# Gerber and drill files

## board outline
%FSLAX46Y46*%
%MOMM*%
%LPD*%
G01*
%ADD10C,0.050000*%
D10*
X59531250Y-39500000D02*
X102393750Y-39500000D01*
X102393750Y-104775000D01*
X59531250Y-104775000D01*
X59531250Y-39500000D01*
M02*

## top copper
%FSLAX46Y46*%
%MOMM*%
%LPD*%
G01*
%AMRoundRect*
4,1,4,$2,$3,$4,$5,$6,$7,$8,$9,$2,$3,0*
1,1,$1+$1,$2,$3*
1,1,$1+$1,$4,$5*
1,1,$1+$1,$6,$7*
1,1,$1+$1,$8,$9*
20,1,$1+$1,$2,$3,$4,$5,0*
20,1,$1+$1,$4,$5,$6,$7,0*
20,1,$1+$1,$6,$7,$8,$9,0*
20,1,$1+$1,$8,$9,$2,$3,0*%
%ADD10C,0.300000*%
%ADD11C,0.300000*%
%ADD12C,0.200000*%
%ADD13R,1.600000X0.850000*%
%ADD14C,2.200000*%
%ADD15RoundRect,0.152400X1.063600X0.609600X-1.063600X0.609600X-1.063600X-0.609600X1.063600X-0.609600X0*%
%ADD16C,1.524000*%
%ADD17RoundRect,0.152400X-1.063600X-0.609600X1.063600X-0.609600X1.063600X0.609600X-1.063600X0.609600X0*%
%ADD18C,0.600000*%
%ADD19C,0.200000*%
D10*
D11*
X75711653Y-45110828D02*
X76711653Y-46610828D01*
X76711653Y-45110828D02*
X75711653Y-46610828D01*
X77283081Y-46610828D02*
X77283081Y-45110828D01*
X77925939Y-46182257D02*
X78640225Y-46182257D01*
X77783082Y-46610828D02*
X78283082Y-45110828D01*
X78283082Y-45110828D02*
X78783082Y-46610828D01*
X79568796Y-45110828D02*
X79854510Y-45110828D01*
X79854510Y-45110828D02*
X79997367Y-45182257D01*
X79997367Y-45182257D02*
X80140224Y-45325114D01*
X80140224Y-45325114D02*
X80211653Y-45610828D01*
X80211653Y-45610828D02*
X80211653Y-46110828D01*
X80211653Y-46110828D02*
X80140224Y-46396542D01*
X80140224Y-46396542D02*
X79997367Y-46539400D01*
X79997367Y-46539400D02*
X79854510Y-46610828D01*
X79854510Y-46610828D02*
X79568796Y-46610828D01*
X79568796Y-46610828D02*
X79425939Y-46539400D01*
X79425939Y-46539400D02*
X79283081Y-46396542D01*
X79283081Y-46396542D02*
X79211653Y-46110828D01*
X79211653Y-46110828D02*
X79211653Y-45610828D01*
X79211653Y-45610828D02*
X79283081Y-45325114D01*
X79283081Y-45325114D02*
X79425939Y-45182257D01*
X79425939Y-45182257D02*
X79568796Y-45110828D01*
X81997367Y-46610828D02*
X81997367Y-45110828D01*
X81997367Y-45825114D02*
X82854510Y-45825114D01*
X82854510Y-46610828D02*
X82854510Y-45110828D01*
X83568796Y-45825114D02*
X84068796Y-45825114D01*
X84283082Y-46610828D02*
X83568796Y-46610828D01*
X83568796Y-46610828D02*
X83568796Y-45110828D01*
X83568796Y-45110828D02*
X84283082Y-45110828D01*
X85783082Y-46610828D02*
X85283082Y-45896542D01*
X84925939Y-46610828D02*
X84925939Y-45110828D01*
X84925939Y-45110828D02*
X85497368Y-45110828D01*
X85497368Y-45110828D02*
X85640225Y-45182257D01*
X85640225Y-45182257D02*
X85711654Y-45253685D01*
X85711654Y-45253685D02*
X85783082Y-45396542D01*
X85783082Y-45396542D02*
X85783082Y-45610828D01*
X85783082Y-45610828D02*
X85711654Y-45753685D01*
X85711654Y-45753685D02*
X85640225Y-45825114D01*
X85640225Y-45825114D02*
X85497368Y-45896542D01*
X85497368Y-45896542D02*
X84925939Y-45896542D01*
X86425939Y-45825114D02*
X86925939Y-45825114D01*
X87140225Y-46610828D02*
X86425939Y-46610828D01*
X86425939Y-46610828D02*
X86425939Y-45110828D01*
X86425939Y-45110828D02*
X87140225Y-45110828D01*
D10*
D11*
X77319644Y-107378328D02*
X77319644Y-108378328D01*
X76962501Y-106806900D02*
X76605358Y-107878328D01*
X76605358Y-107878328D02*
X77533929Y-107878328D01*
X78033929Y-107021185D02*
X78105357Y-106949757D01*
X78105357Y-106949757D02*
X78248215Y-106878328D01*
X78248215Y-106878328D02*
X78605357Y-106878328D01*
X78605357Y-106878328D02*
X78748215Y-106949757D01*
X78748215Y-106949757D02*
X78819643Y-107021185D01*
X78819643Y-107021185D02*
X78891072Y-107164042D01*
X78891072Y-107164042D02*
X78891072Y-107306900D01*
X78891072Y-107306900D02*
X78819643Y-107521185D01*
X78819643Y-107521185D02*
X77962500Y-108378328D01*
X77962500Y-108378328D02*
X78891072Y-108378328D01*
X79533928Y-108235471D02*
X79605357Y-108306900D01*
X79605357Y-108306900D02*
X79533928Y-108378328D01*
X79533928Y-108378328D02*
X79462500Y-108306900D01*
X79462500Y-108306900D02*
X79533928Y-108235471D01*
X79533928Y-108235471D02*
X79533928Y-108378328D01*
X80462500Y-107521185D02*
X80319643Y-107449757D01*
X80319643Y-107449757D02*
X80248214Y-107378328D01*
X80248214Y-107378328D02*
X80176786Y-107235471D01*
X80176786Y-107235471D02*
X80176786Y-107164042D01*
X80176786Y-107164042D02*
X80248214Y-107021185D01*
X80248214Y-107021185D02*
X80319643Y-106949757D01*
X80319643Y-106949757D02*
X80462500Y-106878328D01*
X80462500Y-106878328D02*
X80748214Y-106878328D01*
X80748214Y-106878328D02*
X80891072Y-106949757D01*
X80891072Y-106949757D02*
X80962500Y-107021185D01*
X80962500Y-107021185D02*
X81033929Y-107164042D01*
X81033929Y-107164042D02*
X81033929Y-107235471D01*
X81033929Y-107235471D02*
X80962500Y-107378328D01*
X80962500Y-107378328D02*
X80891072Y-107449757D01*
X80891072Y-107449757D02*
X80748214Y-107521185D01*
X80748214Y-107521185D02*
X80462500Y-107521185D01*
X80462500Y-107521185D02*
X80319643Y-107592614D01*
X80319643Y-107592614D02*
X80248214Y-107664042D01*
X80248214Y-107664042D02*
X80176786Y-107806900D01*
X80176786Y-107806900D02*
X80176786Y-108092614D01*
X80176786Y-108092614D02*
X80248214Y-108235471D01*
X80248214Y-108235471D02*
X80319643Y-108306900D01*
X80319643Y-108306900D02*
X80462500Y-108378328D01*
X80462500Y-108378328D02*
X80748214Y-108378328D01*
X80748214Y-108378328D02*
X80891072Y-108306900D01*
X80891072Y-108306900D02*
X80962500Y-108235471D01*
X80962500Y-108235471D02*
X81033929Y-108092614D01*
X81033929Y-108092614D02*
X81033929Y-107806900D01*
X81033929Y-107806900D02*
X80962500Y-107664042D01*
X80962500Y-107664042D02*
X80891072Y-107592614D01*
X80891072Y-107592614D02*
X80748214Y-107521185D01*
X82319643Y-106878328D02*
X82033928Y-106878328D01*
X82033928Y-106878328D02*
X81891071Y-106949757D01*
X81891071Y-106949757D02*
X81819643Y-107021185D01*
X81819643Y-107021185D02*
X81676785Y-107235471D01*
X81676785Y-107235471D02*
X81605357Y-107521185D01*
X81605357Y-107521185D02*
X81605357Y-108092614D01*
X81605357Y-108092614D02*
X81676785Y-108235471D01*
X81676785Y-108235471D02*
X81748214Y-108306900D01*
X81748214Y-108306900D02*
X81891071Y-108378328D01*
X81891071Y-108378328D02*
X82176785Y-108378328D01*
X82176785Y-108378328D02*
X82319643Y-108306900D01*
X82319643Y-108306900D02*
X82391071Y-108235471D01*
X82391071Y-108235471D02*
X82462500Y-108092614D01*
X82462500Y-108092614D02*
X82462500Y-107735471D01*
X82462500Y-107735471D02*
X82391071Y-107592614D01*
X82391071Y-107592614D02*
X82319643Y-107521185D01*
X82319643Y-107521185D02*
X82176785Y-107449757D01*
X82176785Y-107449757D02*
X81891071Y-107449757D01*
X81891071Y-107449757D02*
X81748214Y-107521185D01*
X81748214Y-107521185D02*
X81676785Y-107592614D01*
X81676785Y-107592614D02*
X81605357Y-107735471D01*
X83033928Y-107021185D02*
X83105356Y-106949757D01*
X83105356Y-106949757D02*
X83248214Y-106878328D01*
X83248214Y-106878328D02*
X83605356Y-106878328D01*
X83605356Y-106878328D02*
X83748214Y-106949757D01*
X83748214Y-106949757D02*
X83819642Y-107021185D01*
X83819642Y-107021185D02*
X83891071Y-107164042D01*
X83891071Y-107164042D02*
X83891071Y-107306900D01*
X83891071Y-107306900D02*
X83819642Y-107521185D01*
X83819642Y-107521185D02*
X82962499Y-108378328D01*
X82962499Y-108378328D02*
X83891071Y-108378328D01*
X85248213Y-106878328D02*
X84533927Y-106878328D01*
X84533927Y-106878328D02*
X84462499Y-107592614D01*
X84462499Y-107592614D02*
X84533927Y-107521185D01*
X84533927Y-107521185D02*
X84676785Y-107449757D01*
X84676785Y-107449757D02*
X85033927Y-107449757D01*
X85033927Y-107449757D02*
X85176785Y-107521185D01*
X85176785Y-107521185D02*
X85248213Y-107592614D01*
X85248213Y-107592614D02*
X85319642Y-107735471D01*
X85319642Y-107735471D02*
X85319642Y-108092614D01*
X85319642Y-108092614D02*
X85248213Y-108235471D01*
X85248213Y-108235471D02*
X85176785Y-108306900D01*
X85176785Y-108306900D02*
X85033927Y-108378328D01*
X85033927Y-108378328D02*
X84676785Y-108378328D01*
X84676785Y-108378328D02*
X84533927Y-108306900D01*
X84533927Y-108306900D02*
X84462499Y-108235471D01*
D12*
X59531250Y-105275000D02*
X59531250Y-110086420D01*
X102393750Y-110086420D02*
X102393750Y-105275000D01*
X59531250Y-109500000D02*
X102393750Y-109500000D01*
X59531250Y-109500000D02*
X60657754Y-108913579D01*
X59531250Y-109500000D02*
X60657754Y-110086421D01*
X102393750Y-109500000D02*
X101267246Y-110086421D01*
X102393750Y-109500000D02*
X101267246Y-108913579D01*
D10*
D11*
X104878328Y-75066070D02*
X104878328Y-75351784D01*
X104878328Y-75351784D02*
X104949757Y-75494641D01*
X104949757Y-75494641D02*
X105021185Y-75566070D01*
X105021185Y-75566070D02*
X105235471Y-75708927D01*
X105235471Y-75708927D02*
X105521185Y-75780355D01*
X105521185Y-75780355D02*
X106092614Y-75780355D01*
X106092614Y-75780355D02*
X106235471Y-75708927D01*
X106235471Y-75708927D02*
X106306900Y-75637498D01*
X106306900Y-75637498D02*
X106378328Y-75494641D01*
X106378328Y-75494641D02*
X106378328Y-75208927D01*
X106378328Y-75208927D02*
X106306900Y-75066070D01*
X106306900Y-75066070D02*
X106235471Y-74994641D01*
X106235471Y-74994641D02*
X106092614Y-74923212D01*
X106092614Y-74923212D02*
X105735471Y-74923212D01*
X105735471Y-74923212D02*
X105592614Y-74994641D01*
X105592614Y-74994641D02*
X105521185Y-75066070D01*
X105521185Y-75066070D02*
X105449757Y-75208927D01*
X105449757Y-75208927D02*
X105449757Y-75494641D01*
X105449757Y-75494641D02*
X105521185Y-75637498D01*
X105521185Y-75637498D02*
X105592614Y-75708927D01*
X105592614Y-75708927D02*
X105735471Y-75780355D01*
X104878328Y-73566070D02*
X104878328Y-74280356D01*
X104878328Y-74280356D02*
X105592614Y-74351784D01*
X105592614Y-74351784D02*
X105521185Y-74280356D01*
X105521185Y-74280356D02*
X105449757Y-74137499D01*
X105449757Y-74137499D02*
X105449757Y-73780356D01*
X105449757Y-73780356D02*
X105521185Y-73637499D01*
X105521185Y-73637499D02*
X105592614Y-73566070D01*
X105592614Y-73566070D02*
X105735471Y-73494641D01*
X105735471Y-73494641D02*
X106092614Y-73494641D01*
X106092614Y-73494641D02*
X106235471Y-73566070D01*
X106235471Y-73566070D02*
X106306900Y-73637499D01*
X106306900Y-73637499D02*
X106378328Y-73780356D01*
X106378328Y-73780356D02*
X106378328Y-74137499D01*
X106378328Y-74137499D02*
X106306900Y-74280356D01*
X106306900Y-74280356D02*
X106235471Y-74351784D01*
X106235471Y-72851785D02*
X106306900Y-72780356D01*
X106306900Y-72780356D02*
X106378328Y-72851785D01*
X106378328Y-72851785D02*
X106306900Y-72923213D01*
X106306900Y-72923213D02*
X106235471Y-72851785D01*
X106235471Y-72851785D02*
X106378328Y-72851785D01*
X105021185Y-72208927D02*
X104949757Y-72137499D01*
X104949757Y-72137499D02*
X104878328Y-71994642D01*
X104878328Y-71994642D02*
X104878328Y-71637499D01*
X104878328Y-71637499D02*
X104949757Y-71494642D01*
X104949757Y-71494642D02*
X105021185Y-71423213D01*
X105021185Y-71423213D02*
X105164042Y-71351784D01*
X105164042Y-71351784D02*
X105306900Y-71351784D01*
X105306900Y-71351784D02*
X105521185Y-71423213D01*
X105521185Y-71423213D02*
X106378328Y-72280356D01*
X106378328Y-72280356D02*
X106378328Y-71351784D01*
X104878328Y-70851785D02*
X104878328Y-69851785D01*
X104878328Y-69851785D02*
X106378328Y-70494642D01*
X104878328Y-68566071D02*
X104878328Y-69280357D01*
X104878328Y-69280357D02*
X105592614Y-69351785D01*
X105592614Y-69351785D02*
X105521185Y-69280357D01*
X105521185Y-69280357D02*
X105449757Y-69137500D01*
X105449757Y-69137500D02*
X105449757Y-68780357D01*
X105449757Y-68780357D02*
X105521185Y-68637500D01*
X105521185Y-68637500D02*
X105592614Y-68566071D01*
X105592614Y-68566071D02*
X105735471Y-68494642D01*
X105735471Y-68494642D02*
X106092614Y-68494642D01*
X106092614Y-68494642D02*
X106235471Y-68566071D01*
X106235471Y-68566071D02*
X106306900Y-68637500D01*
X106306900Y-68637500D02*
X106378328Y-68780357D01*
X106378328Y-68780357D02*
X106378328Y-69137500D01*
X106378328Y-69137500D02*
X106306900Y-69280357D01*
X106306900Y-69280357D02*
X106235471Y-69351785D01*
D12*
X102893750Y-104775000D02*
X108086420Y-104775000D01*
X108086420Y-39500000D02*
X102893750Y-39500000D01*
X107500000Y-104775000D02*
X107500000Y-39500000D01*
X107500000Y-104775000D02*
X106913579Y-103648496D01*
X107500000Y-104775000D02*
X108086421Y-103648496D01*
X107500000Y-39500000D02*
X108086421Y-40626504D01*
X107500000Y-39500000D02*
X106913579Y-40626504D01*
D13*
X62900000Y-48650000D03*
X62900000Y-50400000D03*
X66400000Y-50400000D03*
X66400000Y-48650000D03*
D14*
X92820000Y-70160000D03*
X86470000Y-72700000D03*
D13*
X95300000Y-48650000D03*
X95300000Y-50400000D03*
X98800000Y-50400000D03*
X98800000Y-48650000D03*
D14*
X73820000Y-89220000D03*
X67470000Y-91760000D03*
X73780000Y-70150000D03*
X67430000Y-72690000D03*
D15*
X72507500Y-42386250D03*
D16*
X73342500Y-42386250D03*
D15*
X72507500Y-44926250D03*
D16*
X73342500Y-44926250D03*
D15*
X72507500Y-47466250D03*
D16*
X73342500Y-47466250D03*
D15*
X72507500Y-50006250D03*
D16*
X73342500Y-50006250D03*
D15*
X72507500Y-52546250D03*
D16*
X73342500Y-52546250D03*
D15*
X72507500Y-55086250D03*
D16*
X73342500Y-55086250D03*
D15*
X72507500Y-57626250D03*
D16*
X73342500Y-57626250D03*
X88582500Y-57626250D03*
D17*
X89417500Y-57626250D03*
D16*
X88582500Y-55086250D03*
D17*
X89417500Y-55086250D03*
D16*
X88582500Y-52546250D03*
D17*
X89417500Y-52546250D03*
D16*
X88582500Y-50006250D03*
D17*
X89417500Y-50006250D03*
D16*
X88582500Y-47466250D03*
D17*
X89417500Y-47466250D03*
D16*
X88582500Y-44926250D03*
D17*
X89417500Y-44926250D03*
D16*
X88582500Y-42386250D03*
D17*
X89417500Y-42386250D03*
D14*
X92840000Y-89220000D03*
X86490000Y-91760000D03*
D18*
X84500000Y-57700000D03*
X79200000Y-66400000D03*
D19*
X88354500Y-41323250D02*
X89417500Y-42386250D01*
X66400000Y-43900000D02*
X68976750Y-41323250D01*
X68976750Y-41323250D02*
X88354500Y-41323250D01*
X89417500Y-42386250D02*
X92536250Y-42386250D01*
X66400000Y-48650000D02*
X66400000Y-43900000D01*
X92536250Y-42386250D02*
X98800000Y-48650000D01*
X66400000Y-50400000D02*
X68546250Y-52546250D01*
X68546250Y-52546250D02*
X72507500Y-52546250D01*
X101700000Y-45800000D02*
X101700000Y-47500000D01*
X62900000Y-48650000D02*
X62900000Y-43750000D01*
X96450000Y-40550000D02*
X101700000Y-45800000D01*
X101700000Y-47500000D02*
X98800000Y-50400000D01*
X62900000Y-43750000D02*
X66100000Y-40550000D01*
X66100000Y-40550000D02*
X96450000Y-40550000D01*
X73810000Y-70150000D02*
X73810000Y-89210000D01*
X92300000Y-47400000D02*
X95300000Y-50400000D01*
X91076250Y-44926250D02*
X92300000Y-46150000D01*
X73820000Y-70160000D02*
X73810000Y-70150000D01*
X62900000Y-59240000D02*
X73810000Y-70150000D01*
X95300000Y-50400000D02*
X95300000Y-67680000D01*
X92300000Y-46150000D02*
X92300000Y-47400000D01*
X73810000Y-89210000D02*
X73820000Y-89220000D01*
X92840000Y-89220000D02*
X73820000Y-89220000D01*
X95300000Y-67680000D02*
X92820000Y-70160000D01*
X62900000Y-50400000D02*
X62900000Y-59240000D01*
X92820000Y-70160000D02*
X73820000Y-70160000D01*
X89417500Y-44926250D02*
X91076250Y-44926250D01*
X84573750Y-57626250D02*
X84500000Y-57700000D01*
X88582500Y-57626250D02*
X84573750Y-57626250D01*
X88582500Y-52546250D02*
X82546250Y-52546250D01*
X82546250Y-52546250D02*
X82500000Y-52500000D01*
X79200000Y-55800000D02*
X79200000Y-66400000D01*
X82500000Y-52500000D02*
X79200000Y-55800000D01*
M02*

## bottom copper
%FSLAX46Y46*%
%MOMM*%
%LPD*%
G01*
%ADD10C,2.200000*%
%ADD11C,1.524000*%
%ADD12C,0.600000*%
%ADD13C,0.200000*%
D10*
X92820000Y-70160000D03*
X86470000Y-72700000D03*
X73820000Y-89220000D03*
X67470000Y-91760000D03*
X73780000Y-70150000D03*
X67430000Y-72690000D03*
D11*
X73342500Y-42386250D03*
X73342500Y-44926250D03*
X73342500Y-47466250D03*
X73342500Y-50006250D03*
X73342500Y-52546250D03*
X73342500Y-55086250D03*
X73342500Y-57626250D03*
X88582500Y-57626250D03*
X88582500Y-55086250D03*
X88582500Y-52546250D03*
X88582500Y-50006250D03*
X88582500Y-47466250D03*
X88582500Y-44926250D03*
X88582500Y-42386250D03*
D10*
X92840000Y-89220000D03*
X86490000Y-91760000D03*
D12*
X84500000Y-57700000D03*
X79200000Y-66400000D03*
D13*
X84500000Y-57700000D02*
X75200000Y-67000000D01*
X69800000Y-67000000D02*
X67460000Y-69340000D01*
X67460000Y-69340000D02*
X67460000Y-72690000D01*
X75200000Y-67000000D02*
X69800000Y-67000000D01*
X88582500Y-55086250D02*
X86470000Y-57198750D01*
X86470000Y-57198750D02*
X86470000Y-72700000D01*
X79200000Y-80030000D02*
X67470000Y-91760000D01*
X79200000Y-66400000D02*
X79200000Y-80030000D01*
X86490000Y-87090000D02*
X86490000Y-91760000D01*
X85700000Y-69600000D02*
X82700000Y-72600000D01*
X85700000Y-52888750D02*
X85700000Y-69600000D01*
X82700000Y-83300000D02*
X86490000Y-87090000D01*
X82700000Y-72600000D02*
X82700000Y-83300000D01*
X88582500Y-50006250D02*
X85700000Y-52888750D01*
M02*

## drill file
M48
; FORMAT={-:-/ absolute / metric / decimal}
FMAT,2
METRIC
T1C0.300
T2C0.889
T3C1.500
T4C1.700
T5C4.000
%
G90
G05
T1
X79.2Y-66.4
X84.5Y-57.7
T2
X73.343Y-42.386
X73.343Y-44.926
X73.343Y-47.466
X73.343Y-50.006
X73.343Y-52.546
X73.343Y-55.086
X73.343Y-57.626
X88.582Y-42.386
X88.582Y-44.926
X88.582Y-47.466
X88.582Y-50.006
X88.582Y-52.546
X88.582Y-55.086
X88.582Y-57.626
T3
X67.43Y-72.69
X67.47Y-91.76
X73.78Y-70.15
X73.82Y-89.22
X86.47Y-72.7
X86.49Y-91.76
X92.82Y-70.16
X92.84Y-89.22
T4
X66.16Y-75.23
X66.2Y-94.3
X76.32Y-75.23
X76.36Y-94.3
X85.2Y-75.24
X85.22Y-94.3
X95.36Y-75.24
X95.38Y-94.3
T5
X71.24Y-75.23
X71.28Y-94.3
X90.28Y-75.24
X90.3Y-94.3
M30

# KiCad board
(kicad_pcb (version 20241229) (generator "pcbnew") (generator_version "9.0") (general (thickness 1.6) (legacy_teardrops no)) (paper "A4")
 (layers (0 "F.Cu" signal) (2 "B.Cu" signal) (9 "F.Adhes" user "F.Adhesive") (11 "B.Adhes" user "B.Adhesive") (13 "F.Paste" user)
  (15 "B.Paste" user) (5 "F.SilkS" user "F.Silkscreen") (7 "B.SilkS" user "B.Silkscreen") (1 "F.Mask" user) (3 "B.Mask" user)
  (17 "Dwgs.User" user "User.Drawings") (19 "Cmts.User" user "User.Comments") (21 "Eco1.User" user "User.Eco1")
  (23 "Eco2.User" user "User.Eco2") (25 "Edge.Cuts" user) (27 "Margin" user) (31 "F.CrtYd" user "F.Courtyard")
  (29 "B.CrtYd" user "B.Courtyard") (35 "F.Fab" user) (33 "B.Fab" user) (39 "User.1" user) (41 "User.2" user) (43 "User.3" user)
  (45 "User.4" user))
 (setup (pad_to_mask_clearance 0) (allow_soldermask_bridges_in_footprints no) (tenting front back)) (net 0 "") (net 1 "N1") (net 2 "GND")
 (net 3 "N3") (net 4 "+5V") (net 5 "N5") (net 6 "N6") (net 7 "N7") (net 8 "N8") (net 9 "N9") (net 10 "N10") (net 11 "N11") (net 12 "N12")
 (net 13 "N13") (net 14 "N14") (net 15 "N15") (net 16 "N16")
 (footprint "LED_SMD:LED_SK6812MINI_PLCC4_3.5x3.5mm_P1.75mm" (layer "F.Cu") (at 64.65 49.525)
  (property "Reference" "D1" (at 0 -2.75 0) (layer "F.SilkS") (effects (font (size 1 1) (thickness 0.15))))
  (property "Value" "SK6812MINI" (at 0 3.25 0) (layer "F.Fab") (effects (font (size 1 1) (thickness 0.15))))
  (pad "1" smd rect (at -1.75 -0.875) (size 1.6 0.85) (layers "F.Cu" "F.Mask" "F.Paste") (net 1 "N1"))
  (pad "2" smd rect (at -1.75 0.875) (size 1.6 0.85) (layers "F.Cu" "F.Mask" "F.Paste") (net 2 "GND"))
  (pad "3" smd rect (at 1.75 0.875) (size 1.6 0.85) (layers "F.Cu" "F.Mask" "F.Paste") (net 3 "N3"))
  (pad "4" smd rect (at 1.75 -0.875) (size 1.6 0.85) (layers "F.Cu" "F.Mask" "F.Paste") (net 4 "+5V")))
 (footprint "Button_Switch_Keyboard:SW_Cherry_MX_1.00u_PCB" (layer "F.Cu") (at 92.82 70.16)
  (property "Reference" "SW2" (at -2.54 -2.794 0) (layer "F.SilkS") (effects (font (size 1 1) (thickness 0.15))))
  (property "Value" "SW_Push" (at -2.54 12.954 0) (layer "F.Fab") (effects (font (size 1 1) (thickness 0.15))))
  (pad "" np_thru_hole circle (at -7.62 5.08) (size 1.7 1.7) (drill 1.7) (layers "*.Cu" "*.Mask"))
  (pad "" np_thru_hole circle (at -2.54 5.08) (size 4 4) (drill 4) (layers "*.Cu" "*.Mask"))
  (pad "" np_thru_hole circle (at 2.54 5.08) (size 1.7 1.7) (drill 1.7) (layers "*.Cu" "*.Mask"))
  (pad "1" thru_hole circle (at 0 0) (size 2.2 2.2) (drill 1.5) (layers "*.Cu" "*.Mask") (remove_unused_layers no) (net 2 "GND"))
  (pad "2" thru_hole circle (at -6.35 2.54) (size 2.2 2.2) (drill 1.5) (layers "*.Cu" "*.Mask") (remove_unused_layers no) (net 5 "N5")))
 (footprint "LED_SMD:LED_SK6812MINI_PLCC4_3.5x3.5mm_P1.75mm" (layer "F.Cu") (at 97.05 49.525)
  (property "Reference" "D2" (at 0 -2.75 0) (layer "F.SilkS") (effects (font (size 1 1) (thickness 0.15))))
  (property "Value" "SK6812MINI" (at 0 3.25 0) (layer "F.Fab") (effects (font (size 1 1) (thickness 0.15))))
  (pad "1" smd rect (at -1.75 -0.875) (size 1.6 0.85) (layers "F.Cu" "F.Mask" "F.Paste") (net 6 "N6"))
  (pad "2" smd rect (at -1.75 0.875) (size 1.6 0.85) (layers "F.Cu" "F.Mask" "F.Paste") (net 2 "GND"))
  (pad "3" smd rect (at 1.75 0.875) (size 1.6 0.85) (layers "F.Cu" "F.Mask" "F.Paste") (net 1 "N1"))
  (pad "4" smd rect (at 1.75 -0.875) (size 1.6 0.85) (layers "F.Cu" "F.Mask" "F.Paste") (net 4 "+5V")))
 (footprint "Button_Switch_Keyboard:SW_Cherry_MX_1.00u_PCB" (layer "F.Cu") (at 73.82 89.22)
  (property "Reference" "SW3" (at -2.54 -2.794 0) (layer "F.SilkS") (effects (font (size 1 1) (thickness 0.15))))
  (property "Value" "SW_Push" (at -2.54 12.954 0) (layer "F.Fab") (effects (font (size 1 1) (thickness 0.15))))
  (pad "" np_thru_hole circle (at -7.62 5.08) (size 1.7 1.7) (drill 1.7) (layers "*.Cu" "*.Mask"))
  (pad "" np_thru_hole circle (at -2.54 5.08) (size 4 4) (drill 4) (layers "*.Cu" "*.Mask"))
  (pad "" np_thru_hole circle (at 2.54 5.08) (size 1.7 1.7) (drill 1.7) (layers "*.Cu" "*.Mask"))
  (pad "1" thru_hole circle (at 0 0) (size 2.2 2.2) (drill 1.5) (layers "*.Cu" "*.Mask") (remove_unused_layers no) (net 2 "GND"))
  (pad "2" thru_hole circle (at -6.35 2.54) (size 2.2 2.2) (drill 1.5) (layers "*.Cu" "*.Mask") (remove_unused_layers no) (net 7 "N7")))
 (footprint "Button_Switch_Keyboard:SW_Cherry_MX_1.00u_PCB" (layer "F.Cu") (at 73.78 70.15)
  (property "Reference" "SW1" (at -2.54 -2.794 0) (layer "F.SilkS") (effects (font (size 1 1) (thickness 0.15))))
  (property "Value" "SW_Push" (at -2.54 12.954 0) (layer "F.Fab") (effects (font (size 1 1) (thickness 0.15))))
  (pad "" np_thru_hole circle (at -7.62 5.08) (size 1.7 1.7) (drill 1.7) (layers "*.Cu" "*.Mask"))
  (pad "" np_thru_hole circle (at -2.54 5.08) (size 4 4) (drill 4) (layers "*.Cu" "*.Mask"))
  (pad "" np_thru_hole circle (at 2.54 5.08) (size 1.7 1.7) (drill 1.7) (layers "*.Cu" "*.Mask"))
  (pad "1" thru_hole circle (at 0 0) (size 2.2 2.2) (drill 1.5) (layers "*.Cu" "*.Mask") (remove_unused_layers no) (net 2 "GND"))
  (pad "2" thru_hole circle (at -6.35 2.54) (size 2.2 2.2) (drill 1.5) (layers "*.Cu" "*.Mask") (remove_unused_layers no) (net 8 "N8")))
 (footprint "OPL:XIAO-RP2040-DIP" (layer "F.Cu") (at 80.9625 50.00625)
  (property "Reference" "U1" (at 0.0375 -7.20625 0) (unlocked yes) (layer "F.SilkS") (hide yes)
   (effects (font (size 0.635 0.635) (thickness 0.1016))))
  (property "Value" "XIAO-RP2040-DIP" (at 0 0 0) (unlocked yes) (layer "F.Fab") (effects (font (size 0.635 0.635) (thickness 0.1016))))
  (pad "1" smd roundrect (at -8.455 -7.62 180) (size 2.432 1.524) (layers "F.Cu" "F.Mask") (roundrect_rratio 0.1) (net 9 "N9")
   (thermal_bridge_angle 45))
  (pad "1" thru_hole circle (at -7.62 -7.62 180) (size 1.524 1.524) (drill 0.889) (layers "*.Cu" "*.Mask") (remove_unused_layers no)
   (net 9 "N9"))
  (pad "2" smd roundrect (at -8.455 -5.08 180) (size 2.432 1.524) (layers "F.Cu" "F.Mask") (roundrect_rratio 0.1) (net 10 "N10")
   (thermal_bridge_angle 45))
  (pad "2" thru_hole circle (at -7.62 -5.08 180) (size 1.524 1.524) (drill 0.889) (layers "*.Cu" "*.Mask") (remove_unused_layers no)
   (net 10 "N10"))
  (pad "3" smd roundrect (at -8.455 -2.54 180) (size 2.432 1.524) (layers "F.Cu" "F.Mask") (roundrect_rratio 0.1) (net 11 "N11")
   (thermal_bridge_angle 45))
  (pad "3" thru_hole circle (at -7.62 -2.54 180) (size 1.524 1.524) (drill 0.889) (layers "*.Cu" "*.Mask") (remove_unused_layers no)
   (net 11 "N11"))
  (pad "4" smd roundrect (at -8.455 0 180) (size 2.432 1.524) (layers "F.Cu" "F.Mask") (roundrect_rratio 0.1) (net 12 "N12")
   (thermal_bridge_angle 45))
  (pad "4" thru_hole circle (at -7.62 0 180) (size 1.524 1.524) (drill 0.889) (layers "*.Cu" "*.Mask") (remove_unused_layers no)
   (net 12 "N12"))
  (pad "5" smd roundrect (at -8.455 2.54 180) (size 2.432 1.524) (layers "F.Cu" "F.Mask") (roundrect_rratio 0.1) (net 3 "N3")
   (thermal_bridge_angle 45))
  (pad "5" thru_hole circle (at -7.62 2.54 180) (size 1.524 1.524) (drill 0.889) (layers "*.Cu" "*.Mask") (remove_unused_layers no)
   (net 3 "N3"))
  (pad "6" smd roundrect (at -8.455 5.08 180) (size 2.432 1.524) (layers "F.Cu" "F.Mask") (roundrect_rratio 0.1) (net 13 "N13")
   (thermal_bridge_angle 45))
  (pad "6" thru_hole circle (at -7.62 5.08 180) (size 1.524 1.524) (drill 0.889) (layers "*.Cu" "*.Mask") (remove_unused_layers no)
   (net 13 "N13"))
  (pad "7" smd roundrect (at -8.455 7.62 180) (size 2.432 1.524) (layers "F.Cu" "F.Mask") (roundrect_rratio 0.1) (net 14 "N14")
   (thermal_bridge_angle 45))
  (pad "7" thru_hole circle (at -7.62 7.62 180) (size 1.524 1.524) (drill 0.889) (layers "*.Cu" "*.Mask") (remove_unused_layers no)
   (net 14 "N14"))
  (pad "8" thru_hole circle (at 7.62 7.62) (size 1.524 1.524) (drill 0.889) (layers "*.Cu" "*.Mask") (remove_unused_layers no) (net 8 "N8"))
  (pad "8" smd roundrect (at 8.455 7.62) (size 2.432 1.524) (layers "F.Cu" "F.Mask") (roundrect_rratio 0.1) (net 8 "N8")
   (thermal_bridge_angle 45))
  (pad "9" thru_hole circle (at 7.62 5.08) (size 1.524 1.524) (drill 0.889) (layers "*.Cu" "*.Mask") (remove_unused_layers no) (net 5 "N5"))
  (pad "9" smd roundrect (at 8.455 5.08) (size 2.432 1.524) (layers "F.Cu" "F.Mask") (roundrect_rratio 0.1) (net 5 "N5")
   (thermal_bridge_angle 45))
  (pad "10" thru_hole circle (at 7.62 2.54) (size 1.524 1.524) (drill 0.889) (layers "*.Cu" "*.Mask") (remove_unused_layers no) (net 7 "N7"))
  (pad "10" smd roundrect (at 8.455 2.54) (size 2.432 1.524) (layers "F.Cu" "F.Mask") (roundrect_rratio 0.1) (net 7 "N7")
   (thermal_bridge_angle 45))
  (pad "11" thru_hole circle (at 7.62 0) (size 1.524 1.524) (drill 0.889) (layers "*.Cu" "*.Mask") (remove_unused_layers no) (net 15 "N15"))
  (pad "11" smd roundrect (at 8.455 0) (size 2.432 1.524) (layers "F.Cu" "F.Mask") (roundrect_rratio 0.1) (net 15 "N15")
   (thermal_bridge_angle 45))
  (pad "12" thru_hole circle (at 7.62 -2.54) (size 1.524 1.524) (drill 0.889) (layers "*.Cu" "*.Mask") (remove_unused_layers no)
   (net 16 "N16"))
  (pad "12" smd roundrect (at 8.455 -2.54) (size 2.432 1.524) (layers "F.Cu" "F.Mask") (roundrect_rratio 0.1) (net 16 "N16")
   (thermal_bridge_angle 45))
  (pad "13" thru_hole circle (at 7.62 -5.08) (size 1.524 1.524) (drill 0.889) (layers "*.Cu" "*.Mask") (remove_unused_layers no)
   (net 2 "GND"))
  (pad "13" smd roundrect (at 8.455 -5.08) (size 2.432 1.524) (layers "F.Cu" "F.Mask") (roundrect_rratio 0.1) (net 2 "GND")
   (thermal_bridge_angle 45))
  (pad "14" thru_hole circle (at 7.62 -7.62) (size 1.524 1.524) (drill 0.889) (layers "*.Cu" "*.Mask") (remove_unused_layers no)
   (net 4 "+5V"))
  (pad "14" smd roundrect (at 8.455 -7.62) (size 2.432 1.524) (layers "F.Cu" "F.Mask") (roundrect_rratio 0.1) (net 4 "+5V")
   (thermal_bridge_angle 45)))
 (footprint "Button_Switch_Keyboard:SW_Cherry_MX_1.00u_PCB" (layer "F.Cu") (at 92.84 89.22)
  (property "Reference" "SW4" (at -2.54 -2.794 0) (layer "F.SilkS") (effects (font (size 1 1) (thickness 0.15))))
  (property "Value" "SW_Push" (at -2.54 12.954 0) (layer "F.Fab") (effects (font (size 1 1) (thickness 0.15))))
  (pad "" np_thru_hole circle (at -7.62 5.08) (size 1.7 1.7) (drill 1.7) (layers "*.Cu" "*.Mask"))
  (pad "" np_thru_hole circle (at -2.54 5.08) (size 4 4) (drill 4) (layers "*.Cu" "*.Mask"))
  (pad "" np_thru_hole circle (at 2.54 5.08) (size 1.7 1.7) (drill 1.7) (layers "*.Cu" "*.Mask"))
  (pad "1" thru_hole circle (at 0 0) (size 2.2 2.2) (drill 1.5) (layers "*.Cu" "*.Mask") (remove_unused_layers no) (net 2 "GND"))
  (pad "2" thru_hole circle (at -6.35 2.54) (size 2.2 2.2) (drill 1.5) (layers "*.Cu" "*.Mask") (remove_unused_layers no) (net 15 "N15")))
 (gr_rect (start 59.53125 39.5) (end 102.39375 104.775) (stroke (width 0.05) (type default)) (fill no) (layer "Edge.Cuts"))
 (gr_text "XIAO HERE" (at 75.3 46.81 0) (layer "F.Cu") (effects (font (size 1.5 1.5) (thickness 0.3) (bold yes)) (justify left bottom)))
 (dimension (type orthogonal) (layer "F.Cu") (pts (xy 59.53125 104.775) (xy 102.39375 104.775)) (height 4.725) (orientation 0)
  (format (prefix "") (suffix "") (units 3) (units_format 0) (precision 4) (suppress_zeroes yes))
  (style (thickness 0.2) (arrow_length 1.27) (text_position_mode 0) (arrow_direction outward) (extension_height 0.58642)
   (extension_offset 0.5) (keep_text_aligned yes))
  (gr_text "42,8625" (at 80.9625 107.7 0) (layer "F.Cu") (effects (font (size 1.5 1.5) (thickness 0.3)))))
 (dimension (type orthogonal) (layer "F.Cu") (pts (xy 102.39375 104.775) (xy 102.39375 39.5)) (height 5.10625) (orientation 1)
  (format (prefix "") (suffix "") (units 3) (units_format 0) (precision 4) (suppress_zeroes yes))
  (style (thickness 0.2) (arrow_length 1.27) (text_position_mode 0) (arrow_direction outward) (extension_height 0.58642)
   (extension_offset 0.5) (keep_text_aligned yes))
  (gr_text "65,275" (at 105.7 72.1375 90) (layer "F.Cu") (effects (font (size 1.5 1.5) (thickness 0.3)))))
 (segment (start 88.3545 41.32325) (end 89.4175 42.38625) (width 0.2) (layer "F.Cu") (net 4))
 (segment (start 66.4 43.9) (end 68.97675 41.32325) (width 0.2) (layer "F.Cu") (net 4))
 (segment (start 68.97675 41.32325) (end 88.3545 41.32325) (width 0.2) (layer "F.Cu") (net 4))
 (segment (start 89.4175 42.38625) (end 92.53625 42.38625) (width 0.2) (layer "F.Cu") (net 4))
 (segment (start 66.4 48.65) (end 66.4 43.9) (width 0.2) (layer "F.Cu") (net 4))
 (segment (start 92.53625 42.38625) (end 98.8 48.65) (width 0.2) (layer "F.Cu") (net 4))
 (segment (start 66.4 50.4) (end 68.54625 52.54625) (width 0.2) (layer "F.Cu") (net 3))
 (segment (start 68.54625 52.54625) (end 72.5075 52.54625) (width 0.2) (layer "F.Cu") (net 3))
 (segment (start 101.7 45.8) (end 101.7 47.5) (width 0.2) (layer "F.Cu") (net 1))
 (segment (start 62.9 48.65) (end 62.9 43.75) (width 0.2) (layer "F.Cu") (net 1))
 (segment (start 96.45 40.55) (end 101.7 45.8) (width 0.2) (layer "F.Cu") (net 1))
 (segment (start 101.7 47.5) (end 98.8 50.4) (width 0.2) (layer "F.Cu") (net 1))
 (segment (start 62.9 43.75) (end 66.1 40.55) (width 0.2) (layer "F.Cu") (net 1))
 (segment (start 66.1 40.55) (end 96.45 40.55) (width 0.2) (layer "F.Cu") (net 1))
 (segment (start 73.81 70.15) (end 73.81 89.21) (width 0.2) (layer "F.Cu") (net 2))
 (segment (start 92.3 47.4) (end 95.3 50.4) (width 0.2) (layer "F.Cu") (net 2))
 (segment (start 91.07625 44.92625) (end 92.3 46.15) (width 0.2) (layer "F.Cu") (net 2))
 (segment (start 73.82 70.16) (end 73.81 70.15) (width 0.2) (layer "F.Cu") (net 2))
 (segment (start 62.9 59.24) (end 73.81 70.15) (width 0.2) (layer "F.Cu") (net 2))
 (segment (start 95.3 50.4) (end 95.3 67.68) (width 0.2) (layer "F.Cu") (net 2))
 (segment (start 92.3 46.15) (end 92.3 47.4) (width 0.2) (layer "F.Cu") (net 2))
 (segment (start 73.81 89.21) (end 73.82 89.22) (width 0.2) (layer "F.Cu") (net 2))
 (segment (start 92.84 89.22) (end 73.82 89.22) (width 0.2) (layer "F.Cu") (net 2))
 (segment (start 95.3 67.68) (end 92.82 70.16) (width 0.2) (layer "F.Cu") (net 2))
 (segment (start 62.9 50.4) (end 62.9 59.24) (width 0.2) (layer "F.Cu") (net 2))
 (segment (start 92.82 70.16) (end 73.82 70.16) (width 0.2) (layer "F.Cu") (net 2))
 (segment (start 89.4175 44.92625) (end 91.07625 44.92625) (width 0.2) (layer "F.Cu") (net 2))
 (segment (start 84.57375 57.62625) (end 84.5 57.7) (width 0.2) (layer "F.Cu") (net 8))
 (segment (start 88.5825 57.62625) (end 84.57375 57.62625) (width 0.2) (layer "F.Cu") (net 8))
 (via (at 84.5 57.7) (size 0.6) (drill 0.3) (layers "F.Cu" "B.Cu") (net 8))
 (segment (start 84.5 57.7) (end 75.2 67) (width 0.2) (layer "B.Cu") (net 8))
 (segment (start 69.8 67) (end 67.46 69.34) (width 0.2) (layer "B.Cu") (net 8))
 (segment (start 67.46 69.34) (end 67.46 72.69) (width 0.2) (layer "B.Cu") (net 8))
 (segment (start 75.2 67) (end 69.8 67) (width 0.2) (layer "B.Cu") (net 8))
 (segment (start 88.5825 55.08625) (end 86.47 57.19875) (width 0.2) (layer "B.Cu") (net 5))
 (segment (start 86.47 57.19875) (end 86.47 72.7) (width 0.2) (layer "B.Cu") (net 5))
 (segment (start 88.5825 52.54625) (end 82.54625 52.54625) (width 0.2) (layer "F.Cu") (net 7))
 (segment (start 82.54625 52.54625) (end 82.5 52.5) (width 0.2) (layer "F.Cu") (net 7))
 (segment (start 79.2 55.8) (end 79.2 66.4) (width 0.2) (layer "F.Cu") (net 7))
 (segment (start 82.5 52.5) (end 79.2 55.8) (width 0.2) (layer "F.Cu") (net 7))
 (via (at 79.2 66.4) (size 0.6) (drill 0.3) (layers "F.Cu" "B.Cu") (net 7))
 (segment (start 79.2 80.03) (end 67.47 91.76) (width 0.2) (layer "B.Cu") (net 7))
 (segment (start 79.2 66.4) (end 79.2 80.03) (width 0.2) (layer "B.Cu") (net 7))
 (segment (start 86.49 87.09) (end 86.49 91.76) (width 0.2) (layer "B.Cu") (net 15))
 (segment (start 85.7 69.6) (end 82.7 72.6) (width 0.2) (layer "B.Cu") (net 15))
 (segment (start 85.7 52.88875) (end 85.7 69.6) (width 0.2) (layer "B.Cu") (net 15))
 (segment (start 82.7 83.3) (end 86.49 87.09) (width 0.2) (layer "B.Cu") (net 15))
 (segment (start 82.7 72.6) (end 82.7 83.3) (width 0.2) (layer "B.Cu") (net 15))
 (segment (start 88.5825 50.00625) (end 85.7 52.88875) (width 0.2) (layer "B.Cu") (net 15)))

